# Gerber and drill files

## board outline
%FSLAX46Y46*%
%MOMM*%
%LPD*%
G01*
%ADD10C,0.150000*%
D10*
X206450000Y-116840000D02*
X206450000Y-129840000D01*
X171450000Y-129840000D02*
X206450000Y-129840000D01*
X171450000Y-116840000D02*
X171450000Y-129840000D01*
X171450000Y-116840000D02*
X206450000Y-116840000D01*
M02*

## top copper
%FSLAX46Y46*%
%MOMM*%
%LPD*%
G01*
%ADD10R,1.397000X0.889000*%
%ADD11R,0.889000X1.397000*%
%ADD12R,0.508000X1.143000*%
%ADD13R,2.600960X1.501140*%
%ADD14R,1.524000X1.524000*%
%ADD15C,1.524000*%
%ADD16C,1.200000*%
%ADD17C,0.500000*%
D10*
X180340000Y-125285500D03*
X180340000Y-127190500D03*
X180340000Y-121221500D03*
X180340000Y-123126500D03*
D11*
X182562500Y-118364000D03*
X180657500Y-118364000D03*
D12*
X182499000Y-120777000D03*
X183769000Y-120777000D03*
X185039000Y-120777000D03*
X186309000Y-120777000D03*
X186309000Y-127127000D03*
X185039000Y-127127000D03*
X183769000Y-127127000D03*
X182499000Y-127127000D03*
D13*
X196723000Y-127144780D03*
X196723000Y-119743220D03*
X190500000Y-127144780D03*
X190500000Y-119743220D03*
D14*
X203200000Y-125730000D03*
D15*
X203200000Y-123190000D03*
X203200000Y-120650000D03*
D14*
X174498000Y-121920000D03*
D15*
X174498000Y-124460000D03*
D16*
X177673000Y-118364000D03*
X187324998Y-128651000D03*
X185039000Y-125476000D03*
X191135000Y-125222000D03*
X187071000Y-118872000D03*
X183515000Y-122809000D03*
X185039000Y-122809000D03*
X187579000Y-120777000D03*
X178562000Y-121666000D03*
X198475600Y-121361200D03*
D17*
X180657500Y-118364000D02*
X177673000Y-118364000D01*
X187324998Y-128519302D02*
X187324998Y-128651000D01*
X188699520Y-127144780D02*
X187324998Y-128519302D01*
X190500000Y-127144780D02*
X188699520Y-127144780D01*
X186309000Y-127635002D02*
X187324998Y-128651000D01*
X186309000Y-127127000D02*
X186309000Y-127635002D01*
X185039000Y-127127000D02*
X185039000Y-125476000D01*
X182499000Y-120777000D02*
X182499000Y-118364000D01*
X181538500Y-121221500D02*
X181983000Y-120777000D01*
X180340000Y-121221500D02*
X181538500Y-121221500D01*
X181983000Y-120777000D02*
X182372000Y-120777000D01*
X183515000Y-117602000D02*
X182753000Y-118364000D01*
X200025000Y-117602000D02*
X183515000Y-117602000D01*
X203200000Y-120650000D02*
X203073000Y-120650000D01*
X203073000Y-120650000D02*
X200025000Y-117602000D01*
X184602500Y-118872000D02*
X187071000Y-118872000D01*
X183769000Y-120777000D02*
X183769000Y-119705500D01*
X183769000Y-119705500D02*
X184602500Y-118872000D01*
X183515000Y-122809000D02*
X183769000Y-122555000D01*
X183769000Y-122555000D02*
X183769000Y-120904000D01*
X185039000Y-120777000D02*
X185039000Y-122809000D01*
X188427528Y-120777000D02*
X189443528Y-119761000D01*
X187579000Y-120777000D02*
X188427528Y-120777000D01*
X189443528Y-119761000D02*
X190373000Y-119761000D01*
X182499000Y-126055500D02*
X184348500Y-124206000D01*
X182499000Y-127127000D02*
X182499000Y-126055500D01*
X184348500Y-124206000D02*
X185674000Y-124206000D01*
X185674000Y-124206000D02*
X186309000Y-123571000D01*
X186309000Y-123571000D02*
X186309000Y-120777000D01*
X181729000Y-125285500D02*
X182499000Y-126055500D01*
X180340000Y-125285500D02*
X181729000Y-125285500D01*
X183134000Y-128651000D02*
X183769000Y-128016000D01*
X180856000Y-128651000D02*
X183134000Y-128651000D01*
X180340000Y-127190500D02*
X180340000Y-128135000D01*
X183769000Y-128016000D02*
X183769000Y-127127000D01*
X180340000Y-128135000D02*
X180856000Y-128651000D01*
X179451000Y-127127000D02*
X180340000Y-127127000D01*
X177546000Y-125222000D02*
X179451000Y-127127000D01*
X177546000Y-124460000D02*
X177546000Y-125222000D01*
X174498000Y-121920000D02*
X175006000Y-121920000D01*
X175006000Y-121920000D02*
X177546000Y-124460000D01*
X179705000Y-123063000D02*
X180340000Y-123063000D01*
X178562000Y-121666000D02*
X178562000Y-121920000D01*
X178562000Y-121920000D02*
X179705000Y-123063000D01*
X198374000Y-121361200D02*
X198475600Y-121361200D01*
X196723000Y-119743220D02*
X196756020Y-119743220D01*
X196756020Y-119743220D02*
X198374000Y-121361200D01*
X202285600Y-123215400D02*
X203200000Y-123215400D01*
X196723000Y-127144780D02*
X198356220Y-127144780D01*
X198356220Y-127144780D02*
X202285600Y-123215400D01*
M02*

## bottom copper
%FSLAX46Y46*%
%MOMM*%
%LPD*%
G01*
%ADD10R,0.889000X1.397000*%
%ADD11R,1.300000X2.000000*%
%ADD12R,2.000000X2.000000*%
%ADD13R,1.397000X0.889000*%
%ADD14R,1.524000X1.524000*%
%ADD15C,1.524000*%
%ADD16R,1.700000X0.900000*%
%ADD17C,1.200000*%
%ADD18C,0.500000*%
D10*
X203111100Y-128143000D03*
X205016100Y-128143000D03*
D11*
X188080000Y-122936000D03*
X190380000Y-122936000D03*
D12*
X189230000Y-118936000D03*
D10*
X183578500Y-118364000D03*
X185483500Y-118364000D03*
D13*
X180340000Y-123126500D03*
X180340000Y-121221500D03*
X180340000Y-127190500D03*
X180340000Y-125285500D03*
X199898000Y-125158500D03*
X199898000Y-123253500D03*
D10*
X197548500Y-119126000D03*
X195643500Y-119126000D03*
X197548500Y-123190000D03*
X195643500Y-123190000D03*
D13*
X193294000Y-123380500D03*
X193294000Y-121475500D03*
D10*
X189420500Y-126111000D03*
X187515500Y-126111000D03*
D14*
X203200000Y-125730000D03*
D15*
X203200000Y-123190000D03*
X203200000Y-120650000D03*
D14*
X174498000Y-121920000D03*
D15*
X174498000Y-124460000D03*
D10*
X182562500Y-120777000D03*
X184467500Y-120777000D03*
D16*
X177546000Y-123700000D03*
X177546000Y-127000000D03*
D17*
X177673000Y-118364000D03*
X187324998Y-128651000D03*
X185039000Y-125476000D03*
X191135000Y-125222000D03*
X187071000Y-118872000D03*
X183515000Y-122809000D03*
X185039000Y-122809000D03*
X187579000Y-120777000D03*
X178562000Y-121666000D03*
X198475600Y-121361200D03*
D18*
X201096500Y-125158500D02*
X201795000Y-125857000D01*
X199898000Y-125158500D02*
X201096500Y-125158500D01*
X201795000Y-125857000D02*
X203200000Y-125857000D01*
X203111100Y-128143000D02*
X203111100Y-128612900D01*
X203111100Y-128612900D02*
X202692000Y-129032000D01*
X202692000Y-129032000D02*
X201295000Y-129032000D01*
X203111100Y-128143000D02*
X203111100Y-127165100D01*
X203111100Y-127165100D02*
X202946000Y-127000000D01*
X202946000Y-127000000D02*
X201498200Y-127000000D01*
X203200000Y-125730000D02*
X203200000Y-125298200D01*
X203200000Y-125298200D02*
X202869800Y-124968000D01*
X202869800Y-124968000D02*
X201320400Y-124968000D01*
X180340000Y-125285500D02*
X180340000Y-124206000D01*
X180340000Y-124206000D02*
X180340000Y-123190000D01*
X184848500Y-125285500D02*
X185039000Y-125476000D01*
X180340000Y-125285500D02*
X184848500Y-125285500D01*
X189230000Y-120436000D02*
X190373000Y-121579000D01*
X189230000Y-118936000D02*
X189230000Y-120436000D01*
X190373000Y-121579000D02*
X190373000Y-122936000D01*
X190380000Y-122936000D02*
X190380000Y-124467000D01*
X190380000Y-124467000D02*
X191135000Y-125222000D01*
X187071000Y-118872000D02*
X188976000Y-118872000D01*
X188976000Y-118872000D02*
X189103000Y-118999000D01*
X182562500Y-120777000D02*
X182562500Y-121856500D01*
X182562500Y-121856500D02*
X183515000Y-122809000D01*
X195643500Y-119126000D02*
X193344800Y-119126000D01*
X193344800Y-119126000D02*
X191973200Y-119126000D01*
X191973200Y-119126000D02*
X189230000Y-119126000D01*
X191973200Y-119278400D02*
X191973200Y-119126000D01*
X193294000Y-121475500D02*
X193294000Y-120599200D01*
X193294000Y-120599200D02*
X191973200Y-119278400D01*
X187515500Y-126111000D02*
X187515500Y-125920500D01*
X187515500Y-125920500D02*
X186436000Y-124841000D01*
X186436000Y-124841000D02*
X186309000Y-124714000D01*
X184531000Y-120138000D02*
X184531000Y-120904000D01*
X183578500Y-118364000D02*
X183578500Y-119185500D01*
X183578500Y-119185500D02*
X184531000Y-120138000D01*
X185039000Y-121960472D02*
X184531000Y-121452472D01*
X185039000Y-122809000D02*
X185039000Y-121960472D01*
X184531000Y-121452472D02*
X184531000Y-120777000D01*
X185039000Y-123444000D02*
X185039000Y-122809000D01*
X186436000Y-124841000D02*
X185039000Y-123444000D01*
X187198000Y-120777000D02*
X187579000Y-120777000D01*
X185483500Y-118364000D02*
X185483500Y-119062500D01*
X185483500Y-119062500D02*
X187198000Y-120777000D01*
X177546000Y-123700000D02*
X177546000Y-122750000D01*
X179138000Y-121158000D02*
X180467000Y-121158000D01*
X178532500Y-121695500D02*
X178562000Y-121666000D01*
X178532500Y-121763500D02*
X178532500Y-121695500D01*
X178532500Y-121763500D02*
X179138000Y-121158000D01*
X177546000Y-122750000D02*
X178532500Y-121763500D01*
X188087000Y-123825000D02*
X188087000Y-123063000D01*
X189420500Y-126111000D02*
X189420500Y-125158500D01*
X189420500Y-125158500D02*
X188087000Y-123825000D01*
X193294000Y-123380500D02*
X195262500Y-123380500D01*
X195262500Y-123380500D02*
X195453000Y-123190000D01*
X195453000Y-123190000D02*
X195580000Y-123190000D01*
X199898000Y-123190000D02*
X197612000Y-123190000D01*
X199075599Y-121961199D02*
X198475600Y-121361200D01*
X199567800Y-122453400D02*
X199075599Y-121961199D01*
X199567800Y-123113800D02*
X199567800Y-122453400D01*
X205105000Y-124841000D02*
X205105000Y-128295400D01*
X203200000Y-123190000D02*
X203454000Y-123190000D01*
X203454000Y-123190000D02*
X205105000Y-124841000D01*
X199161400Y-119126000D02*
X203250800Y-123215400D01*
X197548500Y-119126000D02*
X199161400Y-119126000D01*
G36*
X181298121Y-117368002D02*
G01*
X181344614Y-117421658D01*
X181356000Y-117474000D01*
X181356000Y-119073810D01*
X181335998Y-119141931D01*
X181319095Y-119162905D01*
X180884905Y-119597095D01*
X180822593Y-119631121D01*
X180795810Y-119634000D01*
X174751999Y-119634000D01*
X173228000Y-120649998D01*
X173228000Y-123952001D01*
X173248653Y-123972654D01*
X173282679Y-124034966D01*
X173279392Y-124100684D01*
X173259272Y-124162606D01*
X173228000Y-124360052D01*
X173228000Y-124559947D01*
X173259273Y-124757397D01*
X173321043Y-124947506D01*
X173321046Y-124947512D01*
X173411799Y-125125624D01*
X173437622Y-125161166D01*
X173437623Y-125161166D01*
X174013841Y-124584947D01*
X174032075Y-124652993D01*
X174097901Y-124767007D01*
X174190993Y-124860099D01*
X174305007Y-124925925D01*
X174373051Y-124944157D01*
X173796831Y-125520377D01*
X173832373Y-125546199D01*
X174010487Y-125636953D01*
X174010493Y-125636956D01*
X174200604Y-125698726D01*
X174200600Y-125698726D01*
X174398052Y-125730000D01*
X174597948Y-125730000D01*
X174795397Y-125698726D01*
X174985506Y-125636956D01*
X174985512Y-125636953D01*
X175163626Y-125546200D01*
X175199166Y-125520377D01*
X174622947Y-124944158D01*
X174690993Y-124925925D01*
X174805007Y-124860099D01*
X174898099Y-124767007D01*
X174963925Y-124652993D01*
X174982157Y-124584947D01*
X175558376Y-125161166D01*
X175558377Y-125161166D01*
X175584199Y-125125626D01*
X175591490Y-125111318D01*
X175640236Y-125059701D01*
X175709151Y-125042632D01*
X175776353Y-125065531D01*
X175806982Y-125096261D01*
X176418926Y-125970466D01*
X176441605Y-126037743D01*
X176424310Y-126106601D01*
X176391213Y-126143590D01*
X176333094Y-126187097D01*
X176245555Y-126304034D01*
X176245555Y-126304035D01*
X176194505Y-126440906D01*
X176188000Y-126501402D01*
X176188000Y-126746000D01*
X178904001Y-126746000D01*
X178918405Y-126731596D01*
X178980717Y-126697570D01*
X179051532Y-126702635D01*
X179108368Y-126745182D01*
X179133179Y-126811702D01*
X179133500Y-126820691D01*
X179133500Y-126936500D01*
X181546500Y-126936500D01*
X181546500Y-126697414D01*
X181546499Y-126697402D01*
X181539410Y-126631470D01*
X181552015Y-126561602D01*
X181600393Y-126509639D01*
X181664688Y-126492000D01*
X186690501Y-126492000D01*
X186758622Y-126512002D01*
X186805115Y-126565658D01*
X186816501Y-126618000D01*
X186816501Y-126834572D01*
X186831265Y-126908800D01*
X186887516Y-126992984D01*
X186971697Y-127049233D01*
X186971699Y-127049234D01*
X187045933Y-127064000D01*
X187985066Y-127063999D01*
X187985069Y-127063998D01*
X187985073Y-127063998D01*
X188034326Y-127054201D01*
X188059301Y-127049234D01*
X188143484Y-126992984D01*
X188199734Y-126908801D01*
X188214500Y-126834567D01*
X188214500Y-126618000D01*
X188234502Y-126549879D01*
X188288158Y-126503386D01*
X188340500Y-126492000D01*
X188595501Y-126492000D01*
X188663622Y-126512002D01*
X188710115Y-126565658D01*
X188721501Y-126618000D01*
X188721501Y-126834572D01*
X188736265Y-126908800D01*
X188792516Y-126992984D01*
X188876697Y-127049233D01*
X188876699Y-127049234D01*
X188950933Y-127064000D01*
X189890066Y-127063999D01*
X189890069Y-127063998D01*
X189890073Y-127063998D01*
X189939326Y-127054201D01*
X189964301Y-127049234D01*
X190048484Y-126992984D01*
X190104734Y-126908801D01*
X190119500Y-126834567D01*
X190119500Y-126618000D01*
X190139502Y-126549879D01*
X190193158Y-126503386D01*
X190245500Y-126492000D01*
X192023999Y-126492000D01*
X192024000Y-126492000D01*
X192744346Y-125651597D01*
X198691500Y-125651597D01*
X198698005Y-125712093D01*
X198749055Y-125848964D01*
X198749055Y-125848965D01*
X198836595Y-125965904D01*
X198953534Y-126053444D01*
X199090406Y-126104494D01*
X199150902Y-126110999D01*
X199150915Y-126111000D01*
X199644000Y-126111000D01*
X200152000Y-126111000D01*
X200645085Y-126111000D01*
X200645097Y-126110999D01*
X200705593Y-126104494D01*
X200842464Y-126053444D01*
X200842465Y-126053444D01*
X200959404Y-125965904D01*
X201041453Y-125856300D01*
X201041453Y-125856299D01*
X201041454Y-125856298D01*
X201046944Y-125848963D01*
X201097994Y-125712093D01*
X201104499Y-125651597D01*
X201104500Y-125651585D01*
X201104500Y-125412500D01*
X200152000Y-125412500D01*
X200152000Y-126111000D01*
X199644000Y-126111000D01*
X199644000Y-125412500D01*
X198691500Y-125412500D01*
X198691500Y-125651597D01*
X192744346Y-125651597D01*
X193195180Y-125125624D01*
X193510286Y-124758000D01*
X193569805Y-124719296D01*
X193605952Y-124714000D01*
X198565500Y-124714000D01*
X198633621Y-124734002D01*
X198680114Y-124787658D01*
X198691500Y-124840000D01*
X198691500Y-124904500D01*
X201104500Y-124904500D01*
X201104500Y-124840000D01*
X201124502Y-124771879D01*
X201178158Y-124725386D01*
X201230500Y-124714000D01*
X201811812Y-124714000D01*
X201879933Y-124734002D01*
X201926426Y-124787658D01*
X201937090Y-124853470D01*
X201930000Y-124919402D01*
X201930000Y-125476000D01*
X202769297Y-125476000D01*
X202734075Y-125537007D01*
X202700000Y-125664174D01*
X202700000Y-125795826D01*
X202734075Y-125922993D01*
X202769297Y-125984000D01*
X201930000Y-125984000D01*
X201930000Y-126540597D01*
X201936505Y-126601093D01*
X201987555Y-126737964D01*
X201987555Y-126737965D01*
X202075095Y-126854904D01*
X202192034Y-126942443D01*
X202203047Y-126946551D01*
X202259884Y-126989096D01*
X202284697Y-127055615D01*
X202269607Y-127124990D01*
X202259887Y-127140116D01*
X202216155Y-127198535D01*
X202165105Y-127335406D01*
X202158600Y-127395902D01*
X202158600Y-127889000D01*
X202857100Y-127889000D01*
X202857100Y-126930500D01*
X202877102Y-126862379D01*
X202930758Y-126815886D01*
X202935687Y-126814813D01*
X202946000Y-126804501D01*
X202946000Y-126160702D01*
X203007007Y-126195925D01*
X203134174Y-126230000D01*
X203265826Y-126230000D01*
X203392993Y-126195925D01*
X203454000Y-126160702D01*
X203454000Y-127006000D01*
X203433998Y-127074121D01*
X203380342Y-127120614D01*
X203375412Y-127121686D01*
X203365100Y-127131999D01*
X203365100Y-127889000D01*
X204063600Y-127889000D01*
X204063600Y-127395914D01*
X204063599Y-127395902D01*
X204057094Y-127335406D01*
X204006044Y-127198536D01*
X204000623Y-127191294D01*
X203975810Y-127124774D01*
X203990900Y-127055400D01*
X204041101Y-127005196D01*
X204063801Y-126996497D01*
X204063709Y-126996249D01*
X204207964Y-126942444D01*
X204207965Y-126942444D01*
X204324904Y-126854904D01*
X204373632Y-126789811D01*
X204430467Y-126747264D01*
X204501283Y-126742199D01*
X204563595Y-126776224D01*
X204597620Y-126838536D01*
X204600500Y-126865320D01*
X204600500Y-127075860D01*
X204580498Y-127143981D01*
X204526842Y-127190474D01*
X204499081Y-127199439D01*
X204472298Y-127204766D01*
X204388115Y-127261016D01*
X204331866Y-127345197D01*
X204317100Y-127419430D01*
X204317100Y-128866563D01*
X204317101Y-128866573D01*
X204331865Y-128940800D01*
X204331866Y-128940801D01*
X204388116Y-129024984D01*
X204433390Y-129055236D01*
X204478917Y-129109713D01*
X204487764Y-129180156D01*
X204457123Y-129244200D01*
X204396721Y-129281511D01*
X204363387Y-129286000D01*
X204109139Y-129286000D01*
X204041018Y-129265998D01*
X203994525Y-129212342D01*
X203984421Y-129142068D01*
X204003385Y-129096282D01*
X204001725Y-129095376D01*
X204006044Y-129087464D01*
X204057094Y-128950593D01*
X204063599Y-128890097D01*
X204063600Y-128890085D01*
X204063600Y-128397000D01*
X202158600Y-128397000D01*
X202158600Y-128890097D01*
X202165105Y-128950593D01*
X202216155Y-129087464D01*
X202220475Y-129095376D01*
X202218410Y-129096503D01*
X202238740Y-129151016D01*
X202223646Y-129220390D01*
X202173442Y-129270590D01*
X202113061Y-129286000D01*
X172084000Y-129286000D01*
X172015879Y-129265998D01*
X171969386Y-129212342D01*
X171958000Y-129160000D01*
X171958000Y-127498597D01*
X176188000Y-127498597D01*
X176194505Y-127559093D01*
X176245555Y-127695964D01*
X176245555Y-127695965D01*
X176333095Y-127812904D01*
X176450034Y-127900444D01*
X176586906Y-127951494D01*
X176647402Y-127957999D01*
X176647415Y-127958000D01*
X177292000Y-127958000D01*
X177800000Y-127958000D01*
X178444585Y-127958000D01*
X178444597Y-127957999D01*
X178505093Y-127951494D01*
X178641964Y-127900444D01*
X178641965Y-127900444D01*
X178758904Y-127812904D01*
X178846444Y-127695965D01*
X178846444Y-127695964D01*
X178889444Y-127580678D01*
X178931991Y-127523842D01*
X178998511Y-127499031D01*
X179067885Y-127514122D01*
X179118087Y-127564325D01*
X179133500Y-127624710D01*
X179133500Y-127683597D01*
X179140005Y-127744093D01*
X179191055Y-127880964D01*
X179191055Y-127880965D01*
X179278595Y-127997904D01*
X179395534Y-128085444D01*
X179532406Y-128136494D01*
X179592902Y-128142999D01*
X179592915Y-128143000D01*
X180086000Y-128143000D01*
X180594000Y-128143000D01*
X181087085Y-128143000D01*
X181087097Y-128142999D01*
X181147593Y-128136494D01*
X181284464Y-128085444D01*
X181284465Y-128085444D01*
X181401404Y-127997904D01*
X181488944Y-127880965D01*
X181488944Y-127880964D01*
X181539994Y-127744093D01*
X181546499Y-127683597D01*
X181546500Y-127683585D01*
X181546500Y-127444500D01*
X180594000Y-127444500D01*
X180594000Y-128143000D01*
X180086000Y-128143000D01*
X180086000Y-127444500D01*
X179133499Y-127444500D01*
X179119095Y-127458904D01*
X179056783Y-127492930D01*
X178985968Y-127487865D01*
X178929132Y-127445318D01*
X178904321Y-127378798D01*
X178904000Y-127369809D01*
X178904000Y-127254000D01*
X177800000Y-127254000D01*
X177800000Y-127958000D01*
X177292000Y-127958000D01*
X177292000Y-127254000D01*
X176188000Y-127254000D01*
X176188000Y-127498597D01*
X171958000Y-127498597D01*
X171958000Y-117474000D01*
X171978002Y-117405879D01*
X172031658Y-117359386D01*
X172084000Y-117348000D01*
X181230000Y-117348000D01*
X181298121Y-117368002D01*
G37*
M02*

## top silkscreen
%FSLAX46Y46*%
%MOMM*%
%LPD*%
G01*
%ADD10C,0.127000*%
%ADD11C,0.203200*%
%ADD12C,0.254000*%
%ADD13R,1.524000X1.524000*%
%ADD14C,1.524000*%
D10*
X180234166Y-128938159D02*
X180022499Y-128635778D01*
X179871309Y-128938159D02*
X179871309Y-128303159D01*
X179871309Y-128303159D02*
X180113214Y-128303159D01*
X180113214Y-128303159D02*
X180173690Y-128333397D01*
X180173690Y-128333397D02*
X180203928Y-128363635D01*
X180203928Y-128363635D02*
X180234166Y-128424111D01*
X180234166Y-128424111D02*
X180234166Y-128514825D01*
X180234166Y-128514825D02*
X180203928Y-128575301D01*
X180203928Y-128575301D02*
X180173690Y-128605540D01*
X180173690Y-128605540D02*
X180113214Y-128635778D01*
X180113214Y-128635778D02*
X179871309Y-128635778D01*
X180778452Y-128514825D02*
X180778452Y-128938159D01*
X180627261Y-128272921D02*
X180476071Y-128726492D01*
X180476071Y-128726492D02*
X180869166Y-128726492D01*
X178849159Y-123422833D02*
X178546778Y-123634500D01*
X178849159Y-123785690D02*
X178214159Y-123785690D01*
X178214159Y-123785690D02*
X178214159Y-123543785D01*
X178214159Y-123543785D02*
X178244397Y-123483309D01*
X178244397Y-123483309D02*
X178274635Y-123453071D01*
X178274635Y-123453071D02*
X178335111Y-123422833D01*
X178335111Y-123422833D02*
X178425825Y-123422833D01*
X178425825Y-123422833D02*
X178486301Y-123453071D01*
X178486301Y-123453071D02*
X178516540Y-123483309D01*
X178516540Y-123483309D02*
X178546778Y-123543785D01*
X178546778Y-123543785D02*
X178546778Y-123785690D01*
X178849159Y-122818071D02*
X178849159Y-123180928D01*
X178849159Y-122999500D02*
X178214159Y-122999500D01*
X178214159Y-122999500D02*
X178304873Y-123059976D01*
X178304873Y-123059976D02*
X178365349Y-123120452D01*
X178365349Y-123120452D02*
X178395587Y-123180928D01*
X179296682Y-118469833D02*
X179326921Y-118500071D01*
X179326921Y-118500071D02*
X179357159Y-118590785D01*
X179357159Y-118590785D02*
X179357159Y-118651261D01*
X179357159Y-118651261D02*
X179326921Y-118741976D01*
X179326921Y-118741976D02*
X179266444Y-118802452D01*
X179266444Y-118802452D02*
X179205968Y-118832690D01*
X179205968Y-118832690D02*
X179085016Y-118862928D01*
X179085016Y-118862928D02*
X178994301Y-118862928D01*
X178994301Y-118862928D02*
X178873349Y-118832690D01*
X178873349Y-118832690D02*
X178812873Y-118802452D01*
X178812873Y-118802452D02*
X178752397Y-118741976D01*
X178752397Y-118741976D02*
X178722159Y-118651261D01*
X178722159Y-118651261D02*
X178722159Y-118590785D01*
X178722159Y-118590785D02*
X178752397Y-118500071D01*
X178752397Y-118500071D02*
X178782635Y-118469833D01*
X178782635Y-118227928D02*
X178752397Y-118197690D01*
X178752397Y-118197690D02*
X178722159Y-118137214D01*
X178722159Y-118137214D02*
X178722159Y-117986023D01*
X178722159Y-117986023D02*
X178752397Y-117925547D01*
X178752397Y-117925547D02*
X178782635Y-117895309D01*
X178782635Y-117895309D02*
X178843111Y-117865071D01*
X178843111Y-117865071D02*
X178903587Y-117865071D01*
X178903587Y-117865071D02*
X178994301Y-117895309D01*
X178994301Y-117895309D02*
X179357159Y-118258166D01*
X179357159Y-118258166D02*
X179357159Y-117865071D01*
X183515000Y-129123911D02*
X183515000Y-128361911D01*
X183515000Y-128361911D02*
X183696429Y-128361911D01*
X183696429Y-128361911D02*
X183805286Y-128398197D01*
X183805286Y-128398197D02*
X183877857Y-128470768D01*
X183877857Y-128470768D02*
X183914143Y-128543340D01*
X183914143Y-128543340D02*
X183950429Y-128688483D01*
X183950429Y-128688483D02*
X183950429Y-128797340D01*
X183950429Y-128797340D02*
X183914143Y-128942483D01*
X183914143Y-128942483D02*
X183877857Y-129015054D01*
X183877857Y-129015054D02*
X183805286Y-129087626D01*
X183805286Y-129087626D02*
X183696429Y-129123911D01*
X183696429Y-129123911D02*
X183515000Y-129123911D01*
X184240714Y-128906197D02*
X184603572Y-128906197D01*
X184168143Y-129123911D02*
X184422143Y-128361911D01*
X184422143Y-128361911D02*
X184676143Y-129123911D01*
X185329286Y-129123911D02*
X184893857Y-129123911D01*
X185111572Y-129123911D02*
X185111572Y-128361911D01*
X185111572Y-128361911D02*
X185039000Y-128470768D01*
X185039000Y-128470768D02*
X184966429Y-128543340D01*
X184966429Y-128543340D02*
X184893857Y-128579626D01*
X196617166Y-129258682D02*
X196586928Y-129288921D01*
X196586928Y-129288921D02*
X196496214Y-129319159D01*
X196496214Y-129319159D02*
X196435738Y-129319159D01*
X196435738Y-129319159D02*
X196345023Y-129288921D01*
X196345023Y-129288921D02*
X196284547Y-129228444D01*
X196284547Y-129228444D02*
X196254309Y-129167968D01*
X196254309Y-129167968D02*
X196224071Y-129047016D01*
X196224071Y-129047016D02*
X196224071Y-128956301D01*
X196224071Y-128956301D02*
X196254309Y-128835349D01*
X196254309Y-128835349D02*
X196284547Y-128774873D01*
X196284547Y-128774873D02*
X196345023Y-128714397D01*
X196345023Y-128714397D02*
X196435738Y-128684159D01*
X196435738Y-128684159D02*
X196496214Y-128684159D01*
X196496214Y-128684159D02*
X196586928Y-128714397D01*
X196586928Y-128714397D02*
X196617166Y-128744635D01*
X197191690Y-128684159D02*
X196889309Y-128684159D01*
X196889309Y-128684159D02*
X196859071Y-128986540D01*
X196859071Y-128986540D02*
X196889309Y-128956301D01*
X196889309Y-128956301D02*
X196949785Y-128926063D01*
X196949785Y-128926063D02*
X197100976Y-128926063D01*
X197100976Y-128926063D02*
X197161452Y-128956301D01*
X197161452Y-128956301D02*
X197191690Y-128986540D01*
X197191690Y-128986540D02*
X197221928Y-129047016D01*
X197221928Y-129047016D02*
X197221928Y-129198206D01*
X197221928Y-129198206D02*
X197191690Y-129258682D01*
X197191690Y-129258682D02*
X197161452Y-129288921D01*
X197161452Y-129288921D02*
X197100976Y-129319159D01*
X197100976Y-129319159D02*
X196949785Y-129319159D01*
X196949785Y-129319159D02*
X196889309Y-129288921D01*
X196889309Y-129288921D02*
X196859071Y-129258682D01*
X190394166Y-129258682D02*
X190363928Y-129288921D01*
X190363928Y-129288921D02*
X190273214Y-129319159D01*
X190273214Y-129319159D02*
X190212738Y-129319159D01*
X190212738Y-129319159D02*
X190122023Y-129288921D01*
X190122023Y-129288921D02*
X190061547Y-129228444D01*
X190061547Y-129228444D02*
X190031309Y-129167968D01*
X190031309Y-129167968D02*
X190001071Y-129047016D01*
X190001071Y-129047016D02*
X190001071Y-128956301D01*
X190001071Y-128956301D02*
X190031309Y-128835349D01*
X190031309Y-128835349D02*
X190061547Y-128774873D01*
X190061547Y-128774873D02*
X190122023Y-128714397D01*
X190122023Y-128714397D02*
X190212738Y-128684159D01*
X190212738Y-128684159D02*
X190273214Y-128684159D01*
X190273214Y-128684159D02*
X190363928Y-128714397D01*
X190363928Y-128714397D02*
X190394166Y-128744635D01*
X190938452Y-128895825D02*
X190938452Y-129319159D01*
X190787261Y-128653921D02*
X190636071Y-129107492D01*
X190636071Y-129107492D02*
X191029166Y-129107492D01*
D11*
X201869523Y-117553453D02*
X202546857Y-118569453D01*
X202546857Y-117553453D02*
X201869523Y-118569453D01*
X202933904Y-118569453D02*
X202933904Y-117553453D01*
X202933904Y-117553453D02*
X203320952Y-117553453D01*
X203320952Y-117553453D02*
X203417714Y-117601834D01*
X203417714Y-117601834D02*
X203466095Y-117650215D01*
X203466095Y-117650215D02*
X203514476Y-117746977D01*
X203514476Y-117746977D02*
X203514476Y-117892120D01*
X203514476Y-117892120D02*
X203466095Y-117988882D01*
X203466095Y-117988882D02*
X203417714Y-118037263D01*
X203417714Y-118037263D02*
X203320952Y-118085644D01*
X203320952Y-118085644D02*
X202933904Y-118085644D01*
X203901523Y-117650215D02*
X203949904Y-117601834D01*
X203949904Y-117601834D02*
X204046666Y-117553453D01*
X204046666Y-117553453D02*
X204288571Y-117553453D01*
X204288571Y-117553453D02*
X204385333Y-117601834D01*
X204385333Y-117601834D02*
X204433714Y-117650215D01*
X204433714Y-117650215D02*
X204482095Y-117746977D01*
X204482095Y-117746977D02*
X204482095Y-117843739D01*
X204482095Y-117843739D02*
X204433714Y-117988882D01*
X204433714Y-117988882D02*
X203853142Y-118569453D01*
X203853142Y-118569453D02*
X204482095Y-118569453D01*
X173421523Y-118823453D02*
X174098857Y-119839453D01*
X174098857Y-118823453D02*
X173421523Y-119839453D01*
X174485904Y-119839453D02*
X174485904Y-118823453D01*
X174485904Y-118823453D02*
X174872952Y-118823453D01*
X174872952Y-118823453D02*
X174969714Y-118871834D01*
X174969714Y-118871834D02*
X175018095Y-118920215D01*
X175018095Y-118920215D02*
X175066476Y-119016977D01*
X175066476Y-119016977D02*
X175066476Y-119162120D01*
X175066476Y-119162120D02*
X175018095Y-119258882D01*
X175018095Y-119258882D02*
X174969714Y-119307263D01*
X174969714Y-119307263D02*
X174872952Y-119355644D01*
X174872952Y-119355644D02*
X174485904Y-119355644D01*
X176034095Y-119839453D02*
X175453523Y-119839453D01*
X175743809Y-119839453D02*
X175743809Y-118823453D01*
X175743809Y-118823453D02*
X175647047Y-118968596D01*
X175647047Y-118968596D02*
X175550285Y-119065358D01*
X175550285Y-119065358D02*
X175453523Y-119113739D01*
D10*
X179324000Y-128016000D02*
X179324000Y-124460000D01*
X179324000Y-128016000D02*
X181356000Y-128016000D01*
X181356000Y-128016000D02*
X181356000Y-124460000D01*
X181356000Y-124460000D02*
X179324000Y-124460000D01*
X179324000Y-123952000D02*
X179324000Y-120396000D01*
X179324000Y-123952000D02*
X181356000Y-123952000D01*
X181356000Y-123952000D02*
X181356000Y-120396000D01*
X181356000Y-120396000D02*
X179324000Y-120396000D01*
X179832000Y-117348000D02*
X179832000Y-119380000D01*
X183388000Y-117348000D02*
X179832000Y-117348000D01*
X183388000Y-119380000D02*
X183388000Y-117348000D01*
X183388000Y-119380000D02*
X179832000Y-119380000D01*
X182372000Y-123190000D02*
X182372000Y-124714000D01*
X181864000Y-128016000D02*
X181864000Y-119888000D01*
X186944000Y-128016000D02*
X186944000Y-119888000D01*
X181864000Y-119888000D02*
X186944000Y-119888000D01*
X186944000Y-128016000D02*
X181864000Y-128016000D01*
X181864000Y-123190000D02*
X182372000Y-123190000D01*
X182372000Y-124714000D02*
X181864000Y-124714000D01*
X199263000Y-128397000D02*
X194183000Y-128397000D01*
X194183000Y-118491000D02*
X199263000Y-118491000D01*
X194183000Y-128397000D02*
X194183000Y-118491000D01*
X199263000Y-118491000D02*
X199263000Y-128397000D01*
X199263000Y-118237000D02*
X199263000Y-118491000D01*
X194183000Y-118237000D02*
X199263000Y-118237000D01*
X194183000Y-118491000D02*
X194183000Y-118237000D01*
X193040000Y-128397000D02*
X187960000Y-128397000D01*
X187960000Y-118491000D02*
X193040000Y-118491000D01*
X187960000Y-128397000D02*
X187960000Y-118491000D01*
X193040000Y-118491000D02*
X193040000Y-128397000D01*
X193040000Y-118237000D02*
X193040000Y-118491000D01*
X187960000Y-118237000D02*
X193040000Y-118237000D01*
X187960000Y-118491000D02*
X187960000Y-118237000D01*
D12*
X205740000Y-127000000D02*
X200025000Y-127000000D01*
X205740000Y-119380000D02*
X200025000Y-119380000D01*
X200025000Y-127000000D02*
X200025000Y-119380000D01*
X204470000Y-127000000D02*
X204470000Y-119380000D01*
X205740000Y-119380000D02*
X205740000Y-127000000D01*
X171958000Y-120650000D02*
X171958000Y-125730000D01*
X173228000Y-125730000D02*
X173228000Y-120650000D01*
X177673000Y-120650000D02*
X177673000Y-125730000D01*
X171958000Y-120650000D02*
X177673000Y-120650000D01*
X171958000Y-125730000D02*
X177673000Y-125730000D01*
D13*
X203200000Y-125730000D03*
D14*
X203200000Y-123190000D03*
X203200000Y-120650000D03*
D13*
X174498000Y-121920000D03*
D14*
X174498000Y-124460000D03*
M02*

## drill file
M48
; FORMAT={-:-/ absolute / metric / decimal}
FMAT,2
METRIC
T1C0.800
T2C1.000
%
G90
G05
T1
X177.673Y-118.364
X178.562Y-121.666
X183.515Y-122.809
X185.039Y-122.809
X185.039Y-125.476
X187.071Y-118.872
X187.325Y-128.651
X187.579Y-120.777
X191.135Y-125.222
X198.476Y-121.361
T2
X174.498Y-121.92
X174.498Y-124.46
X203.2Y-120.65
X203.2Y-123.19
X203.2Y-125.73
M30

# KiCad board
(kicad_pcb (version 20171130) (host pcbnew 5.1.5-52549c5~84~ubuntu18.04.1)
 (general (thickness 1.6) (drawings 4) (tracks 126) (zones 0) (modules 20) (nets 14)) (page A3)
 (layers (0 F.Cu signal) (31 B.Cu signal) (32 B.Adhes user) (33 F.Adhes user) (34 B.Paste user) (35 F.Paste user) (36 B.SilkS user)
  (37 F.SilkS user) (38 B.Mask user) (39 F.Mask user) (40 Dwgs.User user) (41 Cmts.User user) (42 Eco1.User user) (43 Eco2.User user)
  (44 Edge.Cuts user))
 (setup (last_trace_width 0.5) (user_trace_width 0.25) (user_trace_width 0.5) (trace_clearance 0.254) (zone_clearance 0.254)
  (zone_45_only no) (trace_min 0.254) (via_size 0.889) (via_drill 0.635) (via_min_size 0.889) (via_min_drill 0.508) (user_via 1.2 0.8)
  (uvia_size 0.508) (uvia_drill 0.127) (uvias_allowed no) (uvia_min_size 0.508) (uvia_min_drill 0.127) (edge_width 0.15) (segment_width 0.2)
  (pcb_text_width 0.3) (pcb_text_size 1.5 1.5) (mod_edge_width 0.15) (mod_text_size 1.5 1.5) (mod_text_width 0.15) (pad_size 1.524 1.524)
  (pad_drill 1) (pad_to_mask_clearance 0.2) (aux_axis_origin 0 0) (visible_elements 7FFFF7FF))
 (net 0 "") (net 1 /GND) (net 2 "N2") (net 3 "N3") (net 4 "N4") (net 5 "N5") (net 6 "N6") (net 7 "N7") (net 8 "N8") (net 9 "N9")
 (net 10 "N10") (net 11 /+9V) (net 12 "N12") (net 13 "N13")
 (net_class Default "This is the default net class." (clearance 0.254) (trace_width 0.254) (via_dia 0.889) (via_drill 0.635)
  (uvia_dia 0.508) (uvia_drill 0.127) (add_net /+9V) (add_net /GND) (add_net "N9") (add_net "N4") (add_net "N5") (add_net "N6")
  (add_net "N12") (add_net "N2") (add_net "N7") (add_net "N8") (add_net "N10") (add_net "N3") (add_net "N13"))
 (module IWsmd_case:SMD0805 (layer B.Cu) (at 204.0636 128.143 180)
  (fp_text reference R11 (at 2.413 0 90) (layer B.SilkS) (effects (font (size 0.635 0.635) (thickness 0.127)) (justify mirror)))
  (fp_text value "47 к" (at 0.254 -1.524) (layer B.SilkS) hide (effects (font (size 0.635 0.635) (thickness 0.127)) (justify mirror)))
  (pad 2 smd rect (at 0.9525 0 180) (size 0.889 1.397) (layers B.Cu B.Paste B.Mask) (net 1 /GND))
  (pad 1 smd rect (at -0.9525 0 180) (size 0.889 1.397) (layers B.Cu B.Paste B.Mask) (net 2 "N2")))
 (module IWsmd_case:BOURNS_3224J (layer B.Cu) (at 189.23 122.936)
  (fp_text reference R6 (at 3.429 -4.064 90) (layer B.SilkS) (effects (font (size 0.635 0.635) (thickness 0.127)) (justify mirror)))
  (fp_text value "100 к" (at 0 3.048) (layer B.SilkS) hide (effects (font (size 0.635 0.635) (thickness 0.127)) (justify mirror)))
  (pad 1 smd rect (at -1.15 0) (size 1.3 2) (layers B.Cu B.Paste B.Mask) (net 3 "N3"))
  (pad 3 smd rect (at 1.15 0) (size 1.3 2) (layers B.Cu B.Paste B.Mask) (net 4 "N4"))
  (pad 2 smd rect (at 0 -4) (size 2 2) (layers B.Cu B.Paste B.Mask) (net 4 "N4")))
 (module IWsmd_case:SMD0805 (layer B.Cu) (at 184.531 118.364)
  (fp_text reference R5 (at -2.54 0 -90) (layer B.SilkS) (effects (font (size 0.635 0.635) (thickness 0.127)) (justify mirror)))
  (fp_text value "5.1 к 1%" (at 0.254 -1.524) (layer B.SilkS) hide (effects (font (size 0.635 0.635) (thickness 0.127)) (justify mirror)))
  (pad 1 smd rect (at -0.9525 0) (size 0.889 1.397) (layers B.Cu B.Paste B.Mask) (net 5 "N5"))
  (pad 2 smd rect (at 0.9525 0) (size 0.889 1.397) (layers B.Cu B.Paste B.Mask) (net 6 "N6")))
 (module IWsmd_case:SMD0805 (layer F.Cu) (at 180.34 126.238 90)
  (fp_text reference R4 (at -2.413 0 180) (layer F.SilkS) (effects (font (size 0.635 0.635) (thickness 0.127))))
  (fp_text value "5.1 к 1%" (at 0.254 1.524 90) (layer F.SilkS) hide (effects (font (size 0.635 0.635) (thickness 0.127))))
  (fp_line (start -1.778 -1.016) (end 1.778 -1.016) (layer F.SilkS) (width 0.127))
  (fp_line (start -1.778 -1.016) (end -1.778 1.016) (layer F.SilkS) (width 0.127))
  (fp_line (start -1.778 1.016) (end 1.778 1.016) (layer F.SilkS) (width 0.127))
  (fp_line (start 1.778 1.016) (end 1.778 -1.016) (layer F.SilkS) (width 0.127))
  (pad 2 smd rect (at 0.9525 0 90) (size 0.889 1.397) (layers F.Cu F.Paste F.Mask) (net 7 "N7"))
  (pad 1 smd rect (at -0.9525 0 90) (size 0.889 1.397) (layers F.Cu F.Paste F.Mask) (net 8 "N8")))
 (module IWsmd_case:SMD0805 (layer B.Cu) (at 180.34 122.174 270)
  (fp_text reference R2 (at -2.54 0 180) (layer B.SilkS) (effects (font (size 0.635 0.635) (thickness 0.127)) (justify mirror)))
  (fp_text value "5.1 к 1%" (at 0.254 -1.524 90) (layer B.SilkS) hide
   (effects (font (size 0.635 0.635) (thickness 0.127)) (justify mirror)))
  (pad 2 smd rect (at 0.9525 0 270) (size 0.889 1.397) (layers B.Cu B.Paste B.Mask) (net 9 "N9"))
  (pad 1 smd rect (at -0.9525 0 270) (size 0.889 1.397) (layers B.Cu B.Paste B.Mask) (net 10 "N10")))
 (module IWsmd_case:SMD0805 (layer F.Cu) (at 180.34 122.174 90)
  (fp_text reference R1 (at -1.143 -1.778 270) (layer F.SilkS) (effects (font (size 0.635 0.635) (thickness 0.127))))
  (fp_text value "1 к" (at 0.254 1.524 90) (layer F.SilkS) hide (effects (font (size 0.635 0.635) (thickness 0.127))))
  (fp_line (start -1.778 -1.016) (end 1.778 -1.016) (layer F.SilkS) (width 0.127))
  (fp_line (start -1.778 -1.016) (end -1.778 1.016) (layer F.SilkS) (width 0.127))
  (fp_line (start -1.778 1.016) (end 1.778 1.016) (layer F.SilkS) (width 0.127))
  (fp_line (start 1.778 1.016) (end 1.778 -1.016) (layer F.SilkS) (width 0.127))
  (pad 2 smd rect (at 0.9525 0 90) (size 0.889 1.397) (layers F.Cu F.Paste F.Mask) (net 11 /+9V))
  (pad 1 smd rect (at -0.9525 0 90) (size 0.889 1.397) (layers F.Cu F.Paste F.Mask) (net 10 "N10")))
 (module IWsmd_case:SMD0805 (layer B.Cu) (at 180.34 126.238 270)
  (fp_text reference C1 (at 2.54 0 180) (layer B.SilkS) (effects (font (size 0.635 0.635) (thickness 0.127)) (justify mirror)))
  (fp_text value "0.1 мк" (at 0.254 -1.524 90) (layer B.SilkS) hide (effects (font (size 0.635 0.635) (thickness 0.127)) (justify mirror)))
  (pad 2 smd rect (at 0.9525 0 270) (size 0.889 1.397) (layers B.Cu B.Paste B.Mask) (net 1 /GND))
  (pad 1 smd rect (at -0.9525 0 270) (size 0.889 1.397) (layers B.Cu B.Paste B.Mask) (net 9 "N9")))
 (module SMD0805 (layer F.Cu) (at 181.61 118.364 180)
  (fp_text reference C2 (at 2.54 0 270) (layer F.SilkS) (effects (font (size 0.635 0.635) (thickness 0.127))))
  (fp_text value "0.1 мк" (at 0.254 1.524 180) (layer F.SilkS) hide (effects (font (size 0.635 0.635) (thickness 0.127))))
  (fp_line (start 1.778 1.016) (end 1.778 -1.016) (layer F.SilkS) (width 0.127))
  (fp_line (start -1.778 1.016) (end 1.778 1.016) (layer F.SilkS) (width 0.127))
  (fp_line (start -1.778 -1.016) (end -1.778 1.016) (layer F.SilkS) (width 0.127))
  (fp_line (start -1.778 -1.016) (end 1.778 -1.016) (layer F.SilkS) (width 0.127))
  (pad 1 smd rect (at -0.9525 0 180) (size 0.889 1.397) (layers F.Cu F.Paste F.Mask) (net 11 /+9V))
  (pad 2 smd rect (at 0.9525 0 180) (size 0.889 1.397) (layers F.Cu F.Paste F.Mask) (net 1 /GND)))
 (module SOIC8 (layer F.Cu) (at 184.404 123.952)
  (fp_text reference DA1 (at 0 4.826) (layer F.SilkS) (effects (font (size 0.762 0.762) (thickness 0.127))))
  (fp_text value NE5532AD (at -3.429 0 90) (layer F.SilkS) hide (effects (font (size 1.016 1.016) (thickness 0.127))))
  (fp_line (start -2.032 -0.762) (end -2.032 0.762) (layer F.SilkS) (width 0.127))
  (fp_line (start -2.54 4.064) (end -2.54 -4.064) (layer F.SilkS) (width 0.127))
  (fp_line (start 2.54 4.064) (end 2.54 -4.064) (layer F.SilkS) (width 0.127))
  (fp_line (start -2.54 -4.064) (end 2.54 -4.064) (layer F.SilkS) (width 0.127))
  (fp_line (start 2.54 4.064) (end -2.54 4.064) (layer F.SilkS) (width 0.127))
  (fp_line (start -2.54 -0.762) (end -2.032 -0.762) (layer F.SilkS) (width 0.127))
  (fp_line (start -2.032 0.762) (end -2.54 0.762) (layer F.SilkS) (width 0.127))
  (pad 8 smd rect (at -1.905 -3.175) (size 0.508 1.143) (layers F.Cu F.Paste F.Mask) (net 11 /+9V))
  (pad 7 smd rect (at -0.635 -3.175) (size 0.508 1.143) (layers F.Cu F.Paste F.Mask) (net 4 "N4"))
  (pad 6 smd rect (at 0.635 -3.175) (size 0.508 1.143) (layers F.Cu F.Paste F.Mask) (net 5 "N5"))
  (pad 5 smd rect (at 1.905 -3.175) (size 0.508 1.143) (layers F.Cu F.Paste F.Mask) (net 7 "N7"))
  (pad 4 smd rect (at 1.905 3.175) (size 0.508 1.143) (layers F.Cu F.Paste F.Mask) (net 1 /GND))
  (pad 3 smd rect (at 0.635 3.175) (size 0.508 1.143) (layers F.Cu F.Paste F.Mask) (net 9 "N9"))
  (pad 2 smd rect (at -0.635 3.175) (size 0.508 1.143) (layers F.Cu F.Paste F.Mask) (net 8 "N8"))
  (pad 1 smd rect (at -1.905 3.175) (size 0.508 1.143) (layers F.Cu F.Paste F.Mask) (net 7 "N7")))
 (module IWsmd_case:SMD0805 (layer B.Cu) (at 199.898 124.206 270)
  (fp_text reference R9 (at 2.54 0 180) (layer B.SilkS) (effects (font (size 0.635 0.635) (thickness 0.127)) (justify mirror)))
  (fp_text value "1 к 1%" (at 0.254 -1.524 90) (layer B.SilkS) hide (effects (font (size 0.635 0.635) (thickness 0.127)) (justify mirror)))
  (pad 2 smd rect (at 0.9525 0 270) (size 0.889 1.397) (layers B.Cu B.Paste B.Mask) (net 1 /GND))
  (pad 1 smd rect (at -0.9525 0 270) (size 0.889 1.397) (layers B.Cu B.Paste B.Mask) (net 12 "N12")))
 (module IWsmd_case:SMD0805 (layer B.Cu) (at 196.596 119.126)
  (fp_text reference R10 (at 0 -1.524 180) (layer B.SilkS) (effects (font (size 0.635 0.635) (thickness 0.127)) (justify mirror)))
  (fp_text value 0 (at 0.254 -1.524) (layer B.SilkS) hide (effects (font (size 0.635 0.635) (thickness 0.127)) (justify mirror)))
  (pad 2 smd rect (at 0.9525 0) (size 0.889 1.397) (layers B.Cu B.Paste B.Mask) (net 2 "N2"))
  (pad 1 smd rect (at -0.9525 0) (size 0.889 1.397) (layers B.Cu B.Paste B.Mask) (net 4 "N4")))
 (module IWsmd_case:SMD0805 (layer B.Cu) (at 196.596 123.19)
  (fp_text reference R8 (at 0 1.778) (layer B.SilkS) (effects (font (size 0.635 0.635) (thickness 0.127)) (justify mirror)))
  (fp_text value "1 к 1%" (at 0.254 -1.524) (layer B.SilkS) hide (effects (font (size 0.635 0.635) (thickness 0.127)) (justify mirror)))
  (pad 2 smd rect (at 0.9525 0) (size 0.889 1.397) (layers B.Cu B.Paste B.Mask) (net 12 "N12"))
  (pad 1 smd rect (at -0.9525 0) (size 0.889 1.397) (layers B.Cu B.Paste B.Mask) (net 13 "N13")))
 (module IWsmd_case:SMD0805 (layer B.Cu) (at 193.294 122.428 270)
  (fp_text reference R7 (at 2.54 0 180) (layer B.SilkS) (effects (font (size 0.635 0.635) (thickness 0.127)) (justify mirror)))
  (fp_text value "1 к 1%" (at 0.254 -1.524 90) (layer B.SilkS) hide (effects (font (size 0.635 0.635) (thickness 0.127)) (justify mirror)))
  (pad 2 smd rect (at 0.9525 0 270) (size 0.889 1.397) (layers B.Cu B.Paste B.Mask) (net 13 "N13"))
  (pad 1 smd rect (at -0.9525 0 270) (size 0.889 1.397) (layers B.Cu B.Paste B.Mask) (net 4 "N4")))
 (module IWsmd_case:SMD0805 (layer B.Cu) (at 188.468 126.111)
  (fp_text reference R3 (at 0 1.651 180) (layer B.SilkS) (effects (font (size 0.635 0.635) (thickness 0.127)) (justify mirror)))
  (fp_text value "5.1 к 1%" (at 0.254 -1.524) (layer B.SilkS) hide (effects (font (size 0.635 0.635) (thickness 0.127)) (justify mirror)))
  (pad 2 smd rect (at 0.9525 0) (size 0.889 1.397) (layers B.Cu B.Paste B.Mask) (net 3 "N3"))
  (pad 1 smd rect (at -0.9525 0) (size 0.889 1.397) (layers B.Cu B.Paste B.Mask) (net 5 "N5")))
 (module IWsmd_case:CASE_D (layer F.Cu) (at 196.723 123.444 270)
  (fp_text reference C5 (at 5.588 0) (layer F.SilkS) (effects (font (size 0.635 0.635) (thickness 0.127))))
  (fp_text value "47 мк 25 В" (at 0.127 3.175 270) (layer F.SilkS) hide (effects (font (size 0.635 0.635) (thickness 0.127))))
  (fp_line (start 4.953 -2.54) (end 4.953 2.54) (layer F.SilkS) (width 0.127))
  (fp_line (start -4.953 2.54) (end -4.953 -2.54) (layer F.SilkS) (width 0.127))
  (fp_line (start 4.953 2.54) (end -4.953 2.54) (layer F.SilkS) (width 0.127))
  (fp_line (start -4.953 -2.54) (end 4.953 -2.54) (layer F.SilkS) (width 0.127))
  (fp_line (start -5.207 -2.54) (end -4.953 -2.54) (layer F.SilkS) (width 0.127))
  (fp_line (start -5.207 2.54) (end -5.207 -2.54) (layer F.SilkS) (width 0.127))
  (fp_line (start -4.953 2.54) (end -5.207 2.54) (layer F.SilkS) (width 0.127))
  (pad 2 smd rect (at 3.70078 0 270) (size 1.50114 2.60096) (layers F.Cu F.Paste F.Mask) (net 2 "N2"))
  (pad 1 smd rect (at -3.70078 0 270) (size 1.50114 2.60096) (layers F.Cu F.Paste F.Mask) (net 12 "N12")))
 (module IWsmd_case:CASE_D (layer F.Cu) (at 190.5 123.444 270)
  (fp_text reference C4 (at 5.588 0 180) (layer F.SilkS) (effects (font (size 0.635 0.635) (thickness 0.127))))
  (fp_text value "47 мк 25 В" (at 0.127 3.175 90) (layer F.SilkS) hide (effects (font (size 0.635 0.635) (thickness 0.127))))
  (fp_line (start 4.953 -2.54) (end 4.953 2.54) (layer F.SilkS) (width 0.127))
  (fp_line (start -4.953 2.54) (end -4.953 -2.54) (layer F.SilkS) (width 0.127))
  (fp_line (start 4.953 2.54) (end -4.953 2.54) (layer F.SilkS) (width 0.127))
  (fp_line (start -4.953 -2.54) (end 4.953 -2.54) (layer F.SilkS) (width 0.127))
  (fp_line (start -5.207 -2.54) (end -4.953 -2.54) (layer F.SilkS) (width 0.127))
  (fp_line (start -5.207 2.54) (end -5.207 -2.54) (layer F.SilkS) (width 0.127))
  (fp_line (start -4.953 2.54) (end -5.207 2.54) (layer F.SilkS) (width 0.127))
  (pad 2 smd rect (at 3.70078 0 270) (size 1.50114 2.60096) (layers F.Cu F.Paste F.Mask) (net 1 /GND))
  (pad 1 smd rect (at -3.70078 0 270) (size 1.50114 2.60096) (layers F.Cu F.Paste F.Mask) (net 6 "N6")))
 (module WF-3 (layer F.Cu) (at 203.2 123.19 90)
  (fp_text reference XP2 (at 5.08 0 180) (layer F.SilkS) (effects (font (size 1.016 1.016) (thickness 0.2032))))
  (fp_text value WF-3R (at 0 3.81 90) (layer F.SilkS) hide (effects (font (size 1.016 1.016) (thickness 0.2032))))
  (fp_line (start -3.81 2.54) (end -3.81 -3.175) (layer F.SilkS) (width 0.254))
  (fp_line (start 3.81 2.54) (end 3.81 -3.175) (layer F.SilkS) (width 0.254))
  (fp_line (start -3.81 -3.175) (end 3.81 -3.175) (layer F.SilkS) (width 0.254))
  (fp_line (start -3.81 1.27) (end 3.81 1.27) (layer F.SilkS) (width 0.254))
  (fp_line (start 3.81 2.54) (end -3.81 2.54) (layer F.SilkS) (width 0.254))
  (pad 1 thru_hole rect (at -2.54 0 90) (size 1.524 1.524) (drill 1) (layers *.Cu *.Mask F.SilkS) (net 1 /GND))
  (pad 2 thru_hole circle (at 0 0 90) (size 1.524 1.524) (drill 1) (layers *.Cu *.Mask F.SilkS) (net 2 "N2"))
  (pad 3 thru_hole circle (at 2.54 0 90) (size 1.524 1.524) (drill 1) (layers *.Cu *.Mask F.SilkS) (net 11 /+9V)))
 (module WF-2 (layer F.Cu) (at 174.498 123.19 270)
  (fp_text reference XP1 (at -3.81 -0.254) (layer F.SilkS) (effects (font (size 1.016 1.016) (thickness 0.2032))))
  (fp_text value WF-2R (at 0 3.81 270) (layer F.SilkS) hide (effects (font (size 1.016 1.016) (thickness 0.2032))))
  (fp_line (start -2.54 2.54) (end 2.54 2.54) (layer F.SilkS) (width 0.254))
  (fp_line (start 2.54 1.27) (end -2.54 1.27) (layer F.SilkS) (width 0.254))
  (fp_line (start -2.54 -3.175) (end 2.54 -3.175) (layer F.SilkS) (width 0.254))
  (fp_line (start -2.54 2.54) (end -2.54 -3.175) (layer F.SilkS) (width 0.254))
  (fp_line (start 2.54 2.54) (end 2.54 -3.175) (layer F.SilkS) (width 0.254))
  (pad 1 thru_hole rect (at -1.27 0 270) (size 1.524 1.524) (drill 1) (layers *.Cu *.Mask F.SilkS) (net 8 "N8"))
  (pad 2 thru_hole circle (at 1.27 0 270) (size 1.524 1.524) (drill 1) (layers *.Cu *.Mask F.SilkS) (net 1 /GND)))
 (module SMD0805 (layer B.Cu) (at 183.515 120.777)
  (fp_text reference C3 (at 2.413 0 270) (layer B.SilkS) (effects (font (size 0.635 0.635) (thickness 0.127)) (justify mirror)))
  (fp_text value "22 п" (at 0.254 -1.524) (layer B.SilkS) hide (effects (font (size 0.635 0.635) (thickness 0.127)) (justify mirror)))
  (pad 1 smd rect (at -0.9525 0) (size 0.889 1.397) (layers B.Cu B.Paste B.Mask) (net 4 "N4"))
  (pad 2 smd rect (at 0.9525 0) (size 0.889 1.397) (layers B.Cu B.Paste B.Mask) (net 5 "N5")))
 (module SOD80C (layer B.Cu) (at 177.546 127 90)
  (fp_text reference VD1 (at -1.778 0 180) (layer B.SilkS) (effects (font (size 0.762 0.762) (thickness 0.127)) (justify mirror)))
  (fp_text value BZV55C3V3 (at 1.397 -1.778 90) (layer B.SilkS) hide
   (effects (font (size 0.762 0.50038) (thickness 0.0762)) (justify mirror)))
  (pad 2 smd rect (at 3.3 0 90) (size 0.9 1.7) (layers B.Cu B.Paste B.Mask) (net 10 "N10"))
  (pad 1 smd rect (at 0 0 90) (size 0.9 1.7) (layers B.Cu B.Paste B.Mask) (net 1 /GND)))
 (gr_line (start 206.45 116.84) (end 206.45 129.84) (angle 90) (layer Edge.Cuts) (width 0.15))
 (gr_line (start 171.45 129.84) (end 206.45 129.84) (angle 90) (layer Edge.Cuts) (width 0.15))
 (gr_line (start 171.45 116.84) (end 171.45 129.84) (angle 90) (layer Edge.Cuts) (width 0.15))
 (gr_line (start 171.45 116.84) (end 206.45 116.84) (angle 90) (layer Edge.Cuts) (width 0.15))
 (segment (start 201.0965 125.1585) (end 201.795 125.857) (width 0.5) (layer B.Cu) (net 1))
 (segment (start 199.898 125.1585) (end 201.0965 125.1585) (width 0.5) (layer B.Cu) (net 1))
 (segment (start 201.795 125.857) (end 203.2 125.857) (width 0.5) (layer B.Cu) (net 1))
 (via (at 177.673 118.364) (size 1.2) (drill 0.8) (layers F.Cu B.Cu) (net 1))
 (segment (start 180.6575 118.364) (end 177.673 118.364) (width 0.5) (layer F.Cu) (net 1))
 (via (at 187.324998 128.651) (size 1.2) (drill 0.8) (layers F.Cu B.Cu) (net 1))
 (segment (start 187.324998 128.519302) (end 187.324998 128.651) (width 0.5) (layer F.Cu) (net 1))
 (segment (start 188.69952 127.14478) (end 187.324998 128.519302) (width 0.5) (layer F.Cu) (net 1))
 (segment (start 190.5 127.14478) (end 188.69952 127.14478) (width 0.5) (layer F.Cu) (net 1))
 (segment (start 186.309 127.635002) (end 187.324998 128.651) (width 0.5) (layer F.Cu) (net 1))
 (segment (start 186.309 127.127) (end 186.309 127.635002) (width 0.5) (layer F.Cu) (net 1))
 (segment (start 203.1111 128.143) (end 203.1111 128.6129) (width 0.5) (layer B.Cu) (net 1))
 (segment (start 203.1111 128.6129) (end 202.692 129.032) (width 0.5) (layer B.Cu) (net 1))
 (segment (start 202.692 129.032) (end 201.295 129.032) (width 0.5) (layer B.Cu) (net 1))
 (segment (start 203.1111 128.143) (end 203.1111 127.1651) (width 0.5) (layer B.Cu) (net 1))
 (segment (start 203.1111 127.1651) (end 202.946 127) (width 0.5) (layer B.Cu) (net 1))
 (segment (start 202.946 127) (end 201.4982 127) (width 0.5) (layer B.Cu) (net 1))
 (segment (start 203.2 125.73) (end 203.2 125.2982) (width 0.5) (layer B.Cu) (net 1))
 (segment (start 203.2 125.2982) (end 202.8698 124.968) (width 0.5) (layer B.Cu) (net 1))
 (segment (start 202.8698 124.968) (end 201.3204 124.968) (width 0.5) (layer B.Cu) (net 1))
 (via (at 185.039 125.476) (size 1.2) (drill 0.8) (layers F.Cu B.Cu) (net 9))
 (segment (start 185.039 127.127) (end 185.039 125.476) (width 0.5) (layer F.Cu) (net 9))
 (segment (start 180.34 125.2855) (end 180.34 124.206) (width 0.5) (layer B.Cu) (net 9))
 (segment (start 180.34 124.206) (end 180.34 123.19) (width 0.5) (layer B.Cu) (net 9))
 (segment (start 184.8485 125.2855) (end 185.039 125.476) (width 0.5) (layer B.Cu) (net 9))
 (segment (start 180.34 125.2855) (end 184.8485 125.2855) (width 0.5) (layer B.Cu) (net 9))
 (segment (start 182.499 120.777) (end 182.499 118.364) (width 0.5) (layer F.Cu) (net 11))
 (segment (start 181.5385 121.2215) (end 181.983 120.777) (width 0.5) (layer F.Cu) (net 11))
 (segment (start 180.34 121.2215) (end 181.5385 121.2215) (width 0.5) (layer F.Cu) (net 11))
 (segment (start 181.983 120.777) (end 182.372 120.777) (width 0.5) (layer F.Cu) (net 11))
 (segment (start 183.515 117.602) (end 182.753 118.364) (width 0.5) (layer F.Cu) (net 11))
 (segment (start 200.025 117.602) (end 183.515 117.602) (width 0.5) (layer F.Cu) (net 11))
 (segment (start 203.2 120.65) (end 203.073 120.65) (width 0.5) (layer F.Cu) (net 11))
 (segment (start 203.073 120.65) (end 200.025 117.602) (width 0.5) (layer F.Cu) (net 11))
 (segment (start 189.23 120.436) (end 190.373 121.579) (width 0.5) (layer B.Cu) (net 4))
 (segment (start 189.23 118.936) (end 189.23 120.436) (width 0.5) (layer B.Cu) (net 4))
 (segment (start 190.373 121.579) (end 190.373 122.936) (width 0.5) (layer B.Cu) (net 4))
 (via (at 191.135 125.222) (size 1.2) (drill 0.8) (layers F.Cu B.Cu) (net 4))
 (segment (start 190.38 122.936) (end 190.38 124.467) (width 0.5) (layer B.Cu) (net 4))
 (segment (start 190.38 124.467) (end 191.135 125.222) (width 0.5) (layer B.Cu) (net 4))
 (via (at 187.071 118.872) (size 1.2) (drill 0.8) (layers F.Cu B.Cu) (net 4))
 (segment (start 184.6025 118.872) (end 187.071 118.872) (width 0.5) (layer F.Cu) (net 4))
 (segment (start 183.769 120.777) (end 183.769 119.7055) (width 0.5) (layer F.Cu) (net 4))
 (segment (start 183.769 119.7055) (end 184.6025 118.872) (width 0.5) (layer F.Cu) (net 4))
 (segment (start 187.071 118.872) (end 188.976 118.872) (width 0.5) (layer B.Cu) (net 4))
 (segment (start 188.976 118.872) (end 189.103 118.999) (width 0.5) (layer B.Cu) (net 4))
 (via (at 183.515 122.809) (size 1.2) (drill 0.8) (layers F.Cu B.Cu) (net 4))
 (segment (start 182.5625 120.777) (end 182.5625 121.8565) (width 0.5) (layer B.Cu) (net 4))
 (segment (start 182.5625 121.8565) (end 183.515 122.809) (width 0.5) (layer B.Cu) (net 4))
 (segment (start 183.515 122.809) (end 183.769 122.555) (width 0.5) (layer F.Cu) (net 4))
 (segment (start 183.769 122.555) (end 183.769 120.904) (width 0.5) (layer F.Cu) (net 4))
 (segment (start 195.6435 119.126) (end 193.3448 119.126) (width 0.5) (layer B.Cu) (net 4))
 (segment (start 193.3448 119.126) (end 191.9732 119.126) (width 0.5) (layer B.Cu) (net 4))
 (segment (start 191.9732 119.126) (end 189.23 119.126) (width 0.5) (layer B.Cu) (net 4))
 (segment (start 191.9732 119.2784) (end 191.9732 119.126) (width 0.5) (layer B.Cu) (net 4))
 (segment (start 193.294 121.4755) (end 193.294 120.5992) (width 0.5) (layer B.Cu) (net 4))
 (segment (start 193.294 120.5992) (end 191.9732 119.2784) (width 0.5) (layer B.Cu) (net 4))
 (via (at 185.039 122.809) (size 1.2) (drill 0.8) (layers F.Cu B.Cu) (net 5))
 (segment (start 185.039 120.777) (end 185.039 122.809) (width 0.5) (layer F.Cu) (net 5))
 (segment (start 187.5155 126.111) (end 187.5155 125.9205) (width 0.5) (layer B.Cu) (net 5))
 (segment (start 187.5155 125.9205) (end 186.436 124.841) (width 0.5) (layer B.Cu) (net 5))
 (segment (start 186.436 124.841) (end 186.309 124.714) (width 0.5) (layer B.Cu) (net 5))
 (segment (start 184.531 120.138) (end 184.531 120.904) (width 0.5) (layer B.Cu) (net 5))
 (segment (start 183.5785 118.364) (end 183.5785 119.1855) (width 0.5) (layer B.Cu) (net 5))
 (segment (start 183.5785 119.1855) (end 184.531 120.138) (width 0.5) (layer B.Cu) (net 5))
 (segment (start 185.039 121.960472) (end 184.531 121.452472) (width 0.5) (layer B.Cu) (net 5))
 (segment (start 185.039 122.809) (end 185.039 121.960472) (width 0.5) (layer B.Cu) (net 5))
 (segment (start 184.531 121.452472) (end 184.531 120.777) (width 0.5) (layer B.Cu) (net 5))
 (segment (start 185.039 123.444) (end 185.039 122.809) (width 0.5) (layer B.Cu) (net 5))
 (segment (start 186.436 124.841) (end 185.039 123.444) (width 0.5) (layer B.Cu) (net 5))
 (via (at 187.579 120.777) (size 1.2) (drill 0.8) (layers F.Cu B.Cu) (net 6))
 (segment (start 188.427528 120.777) (end 189.443528 119.761) (width 0.5) (layer F.Cu) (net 6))
 (segment (start 187.579 120.777) (end 188.427528 120.777) (width 0.5) (layer F.Cu) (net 6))
 (segment (start 189.443528 119.761) (end 190.373 119.761) (width 0.5) (layer F.Cu) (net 6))
 (segment (start 187.198 120.777) (end 187.579 120.777) (width 0.5) (layer B.Cu) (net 6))
 (segment (start 185.4835 118.364) (end 185.4835 119.0625) (width 0.5) (layer B.Cu) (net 6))
 (segment (start 185.4835 119.0625) (end 187.198 120.777) (width 0.5) (layer B.Cu) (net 6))
 (segment (start 182.499 126.0555) (end 184.3485 124.206) (width 0.5) (layer F.Cu) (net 7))
 (segment (start 182.499 127.127) (end 182.499 126.0555) (width 0.5) (layer F.Cu) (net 7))
 (segment (start 184.3485 124.206) (end 185.674 124.206) (width 0.5) (layer F.Cu) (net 7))
 (segment (start 185.674 124.206) (end 186.309 123.571) (width 0.5) (layer F.Cu) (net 7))
 (segment (start 186.309 123.571) (end 186.309 120.777) (width 0.5) (layer F.Cu) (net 7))
 (segment (start 181.729 125.2855) (end 182.499 126.0555) (width 0.5) (layer F.Cu) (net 7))
 (segment (start 180.34 125.2855) (end 181.729 125.2855) (width 0.5) (layer F.Cu) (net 7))
 (segment (start 183.134 128.651) (end 183.769 128.016) (width 0.5) (layer F.Cu) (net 8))
 (segment (start 180.856 128.651) (end 183.134 128.651) (width 0.5) (layer F.Cu) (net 8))
 (segment (start 180.34 127.1905) (end 180.34 128.135) (width 0.5) (layer F.Cu) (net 8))
 (segment (start 183.769 128.016) (end 183.769 127.127) (width 0.5) (layer F.Cu) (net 8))
 (segment (start 180.34 128.135) (end 180.856 128.651) (width 0.5) (layer F.Cu) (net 8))
 (segment (start 179.451 127.127) (end 180.34 127.127) (width 0.5) (layer F.Cu) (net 8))
 (segment (start 177.546 125.222) (end 179.451 127.127) (width 0.5) (layer F.Cu) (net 8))
 (segment (start 177.546 124.46) (end 177.546 125.222) (width 0.5) (layer F.Cu) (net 8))
 (segment (start 174.498 121.92) (end 175.006 121.92) (width 0.5) (layer F.Cu) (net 8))
 (segment (start 175.006 121.92) (end 177.546 124.46) (width 0.5) (layer F.Cu) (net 8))
 (segment (start 177.546 123.7) (end 177.546 122.75) (width 0.5) (layer B.Cu) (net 10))
 (segment (start 179.138 121.158) (end 180.467 121.158) (width 0.5) (layer B.Cu) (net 10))
 (via (at 178.562 121.666) (size 1.2) (drill 0.8) (layers F.Cu B.Cu) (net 10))
 (segment (start 178.5325 121.6955) (end 178.562 121.666) (width 0.5) (layer B.Cu) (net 10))
 (segment (start 178.5325 121.7635) (end 178.5325 121.6955) (width 0.5) (layer B.Cu) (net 10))
 (segment (start 178.5325 121.7635) (end 179.138 121.158) (width 0.5) (layer B.Cu) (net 10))
 (segment (start 177.546 122.75) (end 178.5325 121.7635) (width 0.5) (layer B.Cu) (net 10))
 (segment (start 179.705 123.063) (end 180.34 123.063) (width 0.5) (layer F.Cu) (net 10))
 (segment (start 178.562 121.666) (end 178.562 121.92) (width 0.5) (layer F.Cu) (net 10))
 (segment (start 178.562 121.92) (end 179.705 123.063) (width 0.5) (layer F.Cu) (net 10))
 (segment (start 188.087 123.825) (end 188.087 123.063) (width 0.5) (layer B.Cu) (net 3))
 (segment (start 189.4205 126.111) (end 189.4205 125.1585) (width 0.5) (layer B.Cu) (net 3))
 (segment (start 189.4205 125.1585) (end 188.087 123.825) (width 0.5) (layer B.Cu) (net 3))
 (segment (start 193.294 123.3805) (end 195.2625 123.3805) (width 0.5) (layer B.Cu) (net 13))
 (segment (start 195.2625 123.3805) (end 195.453 123.19) (width 0.5) (layer B.Cu) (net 13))
 (segment (start 195.453 123.19) (end 195.58 123.19) (width 0.5) (layer B.Cu) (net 13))
 (segment (start 199.898 123.19) (end 197.612 123.19) (width 0.5) (layer B.Cu) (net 12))
 (segment (start 199.075599 121.961199) (end 198.4756 121.3612) (width 0.5) (layer B.Cu) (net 12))
 (segment (start 199.5678 122.4534) (end 199.075599 121.961199) (width 0.5) (layer B.Cu) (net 12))
 (via (at 198.4756 121.3612) (size 1.2) (drill 0.8) (layers F.Cu B.Cu) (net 12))
 (segment (start 199.5678 123.1138) (end 199.5678 122.4534) (width 0.5) (layer B.Cu) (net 12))
 (segment (start 198.374 121.3612) (end 198.4756 121.3612) (width 0.5) (layer F.Cu) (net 12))
 (segment (start 196.723 119.74322) (end 196.75602 119.74322) (width 0.5) (layer F.Cu) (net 12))
 (segment (start 196.75602 119.74322) (end 198.374 121.3612) (width 0.5) (layer F.Cu) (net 12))
 (segment (start 202.2856 123.2154) (end 203.2 123.2154) (width 0.5) (layer F.Cu) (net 2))
 (segment (start 196.723 127.14478) (end 198.35622 127.14478) (width 0.5) (layer F.Cu) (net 2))
 (segment (start 198.35622 127.14478) (end 202.2856 123.2154) (width 0.5) (layer F.Cu) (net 2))
 (segment (start 205.105 124.841) (end 205.105 128.2954) (width 0.5) (layer B.Cu) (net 2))
 (segment (start 203.2 123.19) (end 203.454 123.19) (width 0.5) (layer B.Cu) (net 2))
 (segment (start 203.454 123.19) (end 205.105 124.841) (width 0.5) (layer B.Cu) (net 2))
 (segment (start 199.1614 119.126) (end 203.2508 123.2154) (width 0.5) (layer B.Cu) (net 2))
 (segment (start 197.5485 119.126) (end 199.1614 119.126) (width 0.5) (layer B.Cu) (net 2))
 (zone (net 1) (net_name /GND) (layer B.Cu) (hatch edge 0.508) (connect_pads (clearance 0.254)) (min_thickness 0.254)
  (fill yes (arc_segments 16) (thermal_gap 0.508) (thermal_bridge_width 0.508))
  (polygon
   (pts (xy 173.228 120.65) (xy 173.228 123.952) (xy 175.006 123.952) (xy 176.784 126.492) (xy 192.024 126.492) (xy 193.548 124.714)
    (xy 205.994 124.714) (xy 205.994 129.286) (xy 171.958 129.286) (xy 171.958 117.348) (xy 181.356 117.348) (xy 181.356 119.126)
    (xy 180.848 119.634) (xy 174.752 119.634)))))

